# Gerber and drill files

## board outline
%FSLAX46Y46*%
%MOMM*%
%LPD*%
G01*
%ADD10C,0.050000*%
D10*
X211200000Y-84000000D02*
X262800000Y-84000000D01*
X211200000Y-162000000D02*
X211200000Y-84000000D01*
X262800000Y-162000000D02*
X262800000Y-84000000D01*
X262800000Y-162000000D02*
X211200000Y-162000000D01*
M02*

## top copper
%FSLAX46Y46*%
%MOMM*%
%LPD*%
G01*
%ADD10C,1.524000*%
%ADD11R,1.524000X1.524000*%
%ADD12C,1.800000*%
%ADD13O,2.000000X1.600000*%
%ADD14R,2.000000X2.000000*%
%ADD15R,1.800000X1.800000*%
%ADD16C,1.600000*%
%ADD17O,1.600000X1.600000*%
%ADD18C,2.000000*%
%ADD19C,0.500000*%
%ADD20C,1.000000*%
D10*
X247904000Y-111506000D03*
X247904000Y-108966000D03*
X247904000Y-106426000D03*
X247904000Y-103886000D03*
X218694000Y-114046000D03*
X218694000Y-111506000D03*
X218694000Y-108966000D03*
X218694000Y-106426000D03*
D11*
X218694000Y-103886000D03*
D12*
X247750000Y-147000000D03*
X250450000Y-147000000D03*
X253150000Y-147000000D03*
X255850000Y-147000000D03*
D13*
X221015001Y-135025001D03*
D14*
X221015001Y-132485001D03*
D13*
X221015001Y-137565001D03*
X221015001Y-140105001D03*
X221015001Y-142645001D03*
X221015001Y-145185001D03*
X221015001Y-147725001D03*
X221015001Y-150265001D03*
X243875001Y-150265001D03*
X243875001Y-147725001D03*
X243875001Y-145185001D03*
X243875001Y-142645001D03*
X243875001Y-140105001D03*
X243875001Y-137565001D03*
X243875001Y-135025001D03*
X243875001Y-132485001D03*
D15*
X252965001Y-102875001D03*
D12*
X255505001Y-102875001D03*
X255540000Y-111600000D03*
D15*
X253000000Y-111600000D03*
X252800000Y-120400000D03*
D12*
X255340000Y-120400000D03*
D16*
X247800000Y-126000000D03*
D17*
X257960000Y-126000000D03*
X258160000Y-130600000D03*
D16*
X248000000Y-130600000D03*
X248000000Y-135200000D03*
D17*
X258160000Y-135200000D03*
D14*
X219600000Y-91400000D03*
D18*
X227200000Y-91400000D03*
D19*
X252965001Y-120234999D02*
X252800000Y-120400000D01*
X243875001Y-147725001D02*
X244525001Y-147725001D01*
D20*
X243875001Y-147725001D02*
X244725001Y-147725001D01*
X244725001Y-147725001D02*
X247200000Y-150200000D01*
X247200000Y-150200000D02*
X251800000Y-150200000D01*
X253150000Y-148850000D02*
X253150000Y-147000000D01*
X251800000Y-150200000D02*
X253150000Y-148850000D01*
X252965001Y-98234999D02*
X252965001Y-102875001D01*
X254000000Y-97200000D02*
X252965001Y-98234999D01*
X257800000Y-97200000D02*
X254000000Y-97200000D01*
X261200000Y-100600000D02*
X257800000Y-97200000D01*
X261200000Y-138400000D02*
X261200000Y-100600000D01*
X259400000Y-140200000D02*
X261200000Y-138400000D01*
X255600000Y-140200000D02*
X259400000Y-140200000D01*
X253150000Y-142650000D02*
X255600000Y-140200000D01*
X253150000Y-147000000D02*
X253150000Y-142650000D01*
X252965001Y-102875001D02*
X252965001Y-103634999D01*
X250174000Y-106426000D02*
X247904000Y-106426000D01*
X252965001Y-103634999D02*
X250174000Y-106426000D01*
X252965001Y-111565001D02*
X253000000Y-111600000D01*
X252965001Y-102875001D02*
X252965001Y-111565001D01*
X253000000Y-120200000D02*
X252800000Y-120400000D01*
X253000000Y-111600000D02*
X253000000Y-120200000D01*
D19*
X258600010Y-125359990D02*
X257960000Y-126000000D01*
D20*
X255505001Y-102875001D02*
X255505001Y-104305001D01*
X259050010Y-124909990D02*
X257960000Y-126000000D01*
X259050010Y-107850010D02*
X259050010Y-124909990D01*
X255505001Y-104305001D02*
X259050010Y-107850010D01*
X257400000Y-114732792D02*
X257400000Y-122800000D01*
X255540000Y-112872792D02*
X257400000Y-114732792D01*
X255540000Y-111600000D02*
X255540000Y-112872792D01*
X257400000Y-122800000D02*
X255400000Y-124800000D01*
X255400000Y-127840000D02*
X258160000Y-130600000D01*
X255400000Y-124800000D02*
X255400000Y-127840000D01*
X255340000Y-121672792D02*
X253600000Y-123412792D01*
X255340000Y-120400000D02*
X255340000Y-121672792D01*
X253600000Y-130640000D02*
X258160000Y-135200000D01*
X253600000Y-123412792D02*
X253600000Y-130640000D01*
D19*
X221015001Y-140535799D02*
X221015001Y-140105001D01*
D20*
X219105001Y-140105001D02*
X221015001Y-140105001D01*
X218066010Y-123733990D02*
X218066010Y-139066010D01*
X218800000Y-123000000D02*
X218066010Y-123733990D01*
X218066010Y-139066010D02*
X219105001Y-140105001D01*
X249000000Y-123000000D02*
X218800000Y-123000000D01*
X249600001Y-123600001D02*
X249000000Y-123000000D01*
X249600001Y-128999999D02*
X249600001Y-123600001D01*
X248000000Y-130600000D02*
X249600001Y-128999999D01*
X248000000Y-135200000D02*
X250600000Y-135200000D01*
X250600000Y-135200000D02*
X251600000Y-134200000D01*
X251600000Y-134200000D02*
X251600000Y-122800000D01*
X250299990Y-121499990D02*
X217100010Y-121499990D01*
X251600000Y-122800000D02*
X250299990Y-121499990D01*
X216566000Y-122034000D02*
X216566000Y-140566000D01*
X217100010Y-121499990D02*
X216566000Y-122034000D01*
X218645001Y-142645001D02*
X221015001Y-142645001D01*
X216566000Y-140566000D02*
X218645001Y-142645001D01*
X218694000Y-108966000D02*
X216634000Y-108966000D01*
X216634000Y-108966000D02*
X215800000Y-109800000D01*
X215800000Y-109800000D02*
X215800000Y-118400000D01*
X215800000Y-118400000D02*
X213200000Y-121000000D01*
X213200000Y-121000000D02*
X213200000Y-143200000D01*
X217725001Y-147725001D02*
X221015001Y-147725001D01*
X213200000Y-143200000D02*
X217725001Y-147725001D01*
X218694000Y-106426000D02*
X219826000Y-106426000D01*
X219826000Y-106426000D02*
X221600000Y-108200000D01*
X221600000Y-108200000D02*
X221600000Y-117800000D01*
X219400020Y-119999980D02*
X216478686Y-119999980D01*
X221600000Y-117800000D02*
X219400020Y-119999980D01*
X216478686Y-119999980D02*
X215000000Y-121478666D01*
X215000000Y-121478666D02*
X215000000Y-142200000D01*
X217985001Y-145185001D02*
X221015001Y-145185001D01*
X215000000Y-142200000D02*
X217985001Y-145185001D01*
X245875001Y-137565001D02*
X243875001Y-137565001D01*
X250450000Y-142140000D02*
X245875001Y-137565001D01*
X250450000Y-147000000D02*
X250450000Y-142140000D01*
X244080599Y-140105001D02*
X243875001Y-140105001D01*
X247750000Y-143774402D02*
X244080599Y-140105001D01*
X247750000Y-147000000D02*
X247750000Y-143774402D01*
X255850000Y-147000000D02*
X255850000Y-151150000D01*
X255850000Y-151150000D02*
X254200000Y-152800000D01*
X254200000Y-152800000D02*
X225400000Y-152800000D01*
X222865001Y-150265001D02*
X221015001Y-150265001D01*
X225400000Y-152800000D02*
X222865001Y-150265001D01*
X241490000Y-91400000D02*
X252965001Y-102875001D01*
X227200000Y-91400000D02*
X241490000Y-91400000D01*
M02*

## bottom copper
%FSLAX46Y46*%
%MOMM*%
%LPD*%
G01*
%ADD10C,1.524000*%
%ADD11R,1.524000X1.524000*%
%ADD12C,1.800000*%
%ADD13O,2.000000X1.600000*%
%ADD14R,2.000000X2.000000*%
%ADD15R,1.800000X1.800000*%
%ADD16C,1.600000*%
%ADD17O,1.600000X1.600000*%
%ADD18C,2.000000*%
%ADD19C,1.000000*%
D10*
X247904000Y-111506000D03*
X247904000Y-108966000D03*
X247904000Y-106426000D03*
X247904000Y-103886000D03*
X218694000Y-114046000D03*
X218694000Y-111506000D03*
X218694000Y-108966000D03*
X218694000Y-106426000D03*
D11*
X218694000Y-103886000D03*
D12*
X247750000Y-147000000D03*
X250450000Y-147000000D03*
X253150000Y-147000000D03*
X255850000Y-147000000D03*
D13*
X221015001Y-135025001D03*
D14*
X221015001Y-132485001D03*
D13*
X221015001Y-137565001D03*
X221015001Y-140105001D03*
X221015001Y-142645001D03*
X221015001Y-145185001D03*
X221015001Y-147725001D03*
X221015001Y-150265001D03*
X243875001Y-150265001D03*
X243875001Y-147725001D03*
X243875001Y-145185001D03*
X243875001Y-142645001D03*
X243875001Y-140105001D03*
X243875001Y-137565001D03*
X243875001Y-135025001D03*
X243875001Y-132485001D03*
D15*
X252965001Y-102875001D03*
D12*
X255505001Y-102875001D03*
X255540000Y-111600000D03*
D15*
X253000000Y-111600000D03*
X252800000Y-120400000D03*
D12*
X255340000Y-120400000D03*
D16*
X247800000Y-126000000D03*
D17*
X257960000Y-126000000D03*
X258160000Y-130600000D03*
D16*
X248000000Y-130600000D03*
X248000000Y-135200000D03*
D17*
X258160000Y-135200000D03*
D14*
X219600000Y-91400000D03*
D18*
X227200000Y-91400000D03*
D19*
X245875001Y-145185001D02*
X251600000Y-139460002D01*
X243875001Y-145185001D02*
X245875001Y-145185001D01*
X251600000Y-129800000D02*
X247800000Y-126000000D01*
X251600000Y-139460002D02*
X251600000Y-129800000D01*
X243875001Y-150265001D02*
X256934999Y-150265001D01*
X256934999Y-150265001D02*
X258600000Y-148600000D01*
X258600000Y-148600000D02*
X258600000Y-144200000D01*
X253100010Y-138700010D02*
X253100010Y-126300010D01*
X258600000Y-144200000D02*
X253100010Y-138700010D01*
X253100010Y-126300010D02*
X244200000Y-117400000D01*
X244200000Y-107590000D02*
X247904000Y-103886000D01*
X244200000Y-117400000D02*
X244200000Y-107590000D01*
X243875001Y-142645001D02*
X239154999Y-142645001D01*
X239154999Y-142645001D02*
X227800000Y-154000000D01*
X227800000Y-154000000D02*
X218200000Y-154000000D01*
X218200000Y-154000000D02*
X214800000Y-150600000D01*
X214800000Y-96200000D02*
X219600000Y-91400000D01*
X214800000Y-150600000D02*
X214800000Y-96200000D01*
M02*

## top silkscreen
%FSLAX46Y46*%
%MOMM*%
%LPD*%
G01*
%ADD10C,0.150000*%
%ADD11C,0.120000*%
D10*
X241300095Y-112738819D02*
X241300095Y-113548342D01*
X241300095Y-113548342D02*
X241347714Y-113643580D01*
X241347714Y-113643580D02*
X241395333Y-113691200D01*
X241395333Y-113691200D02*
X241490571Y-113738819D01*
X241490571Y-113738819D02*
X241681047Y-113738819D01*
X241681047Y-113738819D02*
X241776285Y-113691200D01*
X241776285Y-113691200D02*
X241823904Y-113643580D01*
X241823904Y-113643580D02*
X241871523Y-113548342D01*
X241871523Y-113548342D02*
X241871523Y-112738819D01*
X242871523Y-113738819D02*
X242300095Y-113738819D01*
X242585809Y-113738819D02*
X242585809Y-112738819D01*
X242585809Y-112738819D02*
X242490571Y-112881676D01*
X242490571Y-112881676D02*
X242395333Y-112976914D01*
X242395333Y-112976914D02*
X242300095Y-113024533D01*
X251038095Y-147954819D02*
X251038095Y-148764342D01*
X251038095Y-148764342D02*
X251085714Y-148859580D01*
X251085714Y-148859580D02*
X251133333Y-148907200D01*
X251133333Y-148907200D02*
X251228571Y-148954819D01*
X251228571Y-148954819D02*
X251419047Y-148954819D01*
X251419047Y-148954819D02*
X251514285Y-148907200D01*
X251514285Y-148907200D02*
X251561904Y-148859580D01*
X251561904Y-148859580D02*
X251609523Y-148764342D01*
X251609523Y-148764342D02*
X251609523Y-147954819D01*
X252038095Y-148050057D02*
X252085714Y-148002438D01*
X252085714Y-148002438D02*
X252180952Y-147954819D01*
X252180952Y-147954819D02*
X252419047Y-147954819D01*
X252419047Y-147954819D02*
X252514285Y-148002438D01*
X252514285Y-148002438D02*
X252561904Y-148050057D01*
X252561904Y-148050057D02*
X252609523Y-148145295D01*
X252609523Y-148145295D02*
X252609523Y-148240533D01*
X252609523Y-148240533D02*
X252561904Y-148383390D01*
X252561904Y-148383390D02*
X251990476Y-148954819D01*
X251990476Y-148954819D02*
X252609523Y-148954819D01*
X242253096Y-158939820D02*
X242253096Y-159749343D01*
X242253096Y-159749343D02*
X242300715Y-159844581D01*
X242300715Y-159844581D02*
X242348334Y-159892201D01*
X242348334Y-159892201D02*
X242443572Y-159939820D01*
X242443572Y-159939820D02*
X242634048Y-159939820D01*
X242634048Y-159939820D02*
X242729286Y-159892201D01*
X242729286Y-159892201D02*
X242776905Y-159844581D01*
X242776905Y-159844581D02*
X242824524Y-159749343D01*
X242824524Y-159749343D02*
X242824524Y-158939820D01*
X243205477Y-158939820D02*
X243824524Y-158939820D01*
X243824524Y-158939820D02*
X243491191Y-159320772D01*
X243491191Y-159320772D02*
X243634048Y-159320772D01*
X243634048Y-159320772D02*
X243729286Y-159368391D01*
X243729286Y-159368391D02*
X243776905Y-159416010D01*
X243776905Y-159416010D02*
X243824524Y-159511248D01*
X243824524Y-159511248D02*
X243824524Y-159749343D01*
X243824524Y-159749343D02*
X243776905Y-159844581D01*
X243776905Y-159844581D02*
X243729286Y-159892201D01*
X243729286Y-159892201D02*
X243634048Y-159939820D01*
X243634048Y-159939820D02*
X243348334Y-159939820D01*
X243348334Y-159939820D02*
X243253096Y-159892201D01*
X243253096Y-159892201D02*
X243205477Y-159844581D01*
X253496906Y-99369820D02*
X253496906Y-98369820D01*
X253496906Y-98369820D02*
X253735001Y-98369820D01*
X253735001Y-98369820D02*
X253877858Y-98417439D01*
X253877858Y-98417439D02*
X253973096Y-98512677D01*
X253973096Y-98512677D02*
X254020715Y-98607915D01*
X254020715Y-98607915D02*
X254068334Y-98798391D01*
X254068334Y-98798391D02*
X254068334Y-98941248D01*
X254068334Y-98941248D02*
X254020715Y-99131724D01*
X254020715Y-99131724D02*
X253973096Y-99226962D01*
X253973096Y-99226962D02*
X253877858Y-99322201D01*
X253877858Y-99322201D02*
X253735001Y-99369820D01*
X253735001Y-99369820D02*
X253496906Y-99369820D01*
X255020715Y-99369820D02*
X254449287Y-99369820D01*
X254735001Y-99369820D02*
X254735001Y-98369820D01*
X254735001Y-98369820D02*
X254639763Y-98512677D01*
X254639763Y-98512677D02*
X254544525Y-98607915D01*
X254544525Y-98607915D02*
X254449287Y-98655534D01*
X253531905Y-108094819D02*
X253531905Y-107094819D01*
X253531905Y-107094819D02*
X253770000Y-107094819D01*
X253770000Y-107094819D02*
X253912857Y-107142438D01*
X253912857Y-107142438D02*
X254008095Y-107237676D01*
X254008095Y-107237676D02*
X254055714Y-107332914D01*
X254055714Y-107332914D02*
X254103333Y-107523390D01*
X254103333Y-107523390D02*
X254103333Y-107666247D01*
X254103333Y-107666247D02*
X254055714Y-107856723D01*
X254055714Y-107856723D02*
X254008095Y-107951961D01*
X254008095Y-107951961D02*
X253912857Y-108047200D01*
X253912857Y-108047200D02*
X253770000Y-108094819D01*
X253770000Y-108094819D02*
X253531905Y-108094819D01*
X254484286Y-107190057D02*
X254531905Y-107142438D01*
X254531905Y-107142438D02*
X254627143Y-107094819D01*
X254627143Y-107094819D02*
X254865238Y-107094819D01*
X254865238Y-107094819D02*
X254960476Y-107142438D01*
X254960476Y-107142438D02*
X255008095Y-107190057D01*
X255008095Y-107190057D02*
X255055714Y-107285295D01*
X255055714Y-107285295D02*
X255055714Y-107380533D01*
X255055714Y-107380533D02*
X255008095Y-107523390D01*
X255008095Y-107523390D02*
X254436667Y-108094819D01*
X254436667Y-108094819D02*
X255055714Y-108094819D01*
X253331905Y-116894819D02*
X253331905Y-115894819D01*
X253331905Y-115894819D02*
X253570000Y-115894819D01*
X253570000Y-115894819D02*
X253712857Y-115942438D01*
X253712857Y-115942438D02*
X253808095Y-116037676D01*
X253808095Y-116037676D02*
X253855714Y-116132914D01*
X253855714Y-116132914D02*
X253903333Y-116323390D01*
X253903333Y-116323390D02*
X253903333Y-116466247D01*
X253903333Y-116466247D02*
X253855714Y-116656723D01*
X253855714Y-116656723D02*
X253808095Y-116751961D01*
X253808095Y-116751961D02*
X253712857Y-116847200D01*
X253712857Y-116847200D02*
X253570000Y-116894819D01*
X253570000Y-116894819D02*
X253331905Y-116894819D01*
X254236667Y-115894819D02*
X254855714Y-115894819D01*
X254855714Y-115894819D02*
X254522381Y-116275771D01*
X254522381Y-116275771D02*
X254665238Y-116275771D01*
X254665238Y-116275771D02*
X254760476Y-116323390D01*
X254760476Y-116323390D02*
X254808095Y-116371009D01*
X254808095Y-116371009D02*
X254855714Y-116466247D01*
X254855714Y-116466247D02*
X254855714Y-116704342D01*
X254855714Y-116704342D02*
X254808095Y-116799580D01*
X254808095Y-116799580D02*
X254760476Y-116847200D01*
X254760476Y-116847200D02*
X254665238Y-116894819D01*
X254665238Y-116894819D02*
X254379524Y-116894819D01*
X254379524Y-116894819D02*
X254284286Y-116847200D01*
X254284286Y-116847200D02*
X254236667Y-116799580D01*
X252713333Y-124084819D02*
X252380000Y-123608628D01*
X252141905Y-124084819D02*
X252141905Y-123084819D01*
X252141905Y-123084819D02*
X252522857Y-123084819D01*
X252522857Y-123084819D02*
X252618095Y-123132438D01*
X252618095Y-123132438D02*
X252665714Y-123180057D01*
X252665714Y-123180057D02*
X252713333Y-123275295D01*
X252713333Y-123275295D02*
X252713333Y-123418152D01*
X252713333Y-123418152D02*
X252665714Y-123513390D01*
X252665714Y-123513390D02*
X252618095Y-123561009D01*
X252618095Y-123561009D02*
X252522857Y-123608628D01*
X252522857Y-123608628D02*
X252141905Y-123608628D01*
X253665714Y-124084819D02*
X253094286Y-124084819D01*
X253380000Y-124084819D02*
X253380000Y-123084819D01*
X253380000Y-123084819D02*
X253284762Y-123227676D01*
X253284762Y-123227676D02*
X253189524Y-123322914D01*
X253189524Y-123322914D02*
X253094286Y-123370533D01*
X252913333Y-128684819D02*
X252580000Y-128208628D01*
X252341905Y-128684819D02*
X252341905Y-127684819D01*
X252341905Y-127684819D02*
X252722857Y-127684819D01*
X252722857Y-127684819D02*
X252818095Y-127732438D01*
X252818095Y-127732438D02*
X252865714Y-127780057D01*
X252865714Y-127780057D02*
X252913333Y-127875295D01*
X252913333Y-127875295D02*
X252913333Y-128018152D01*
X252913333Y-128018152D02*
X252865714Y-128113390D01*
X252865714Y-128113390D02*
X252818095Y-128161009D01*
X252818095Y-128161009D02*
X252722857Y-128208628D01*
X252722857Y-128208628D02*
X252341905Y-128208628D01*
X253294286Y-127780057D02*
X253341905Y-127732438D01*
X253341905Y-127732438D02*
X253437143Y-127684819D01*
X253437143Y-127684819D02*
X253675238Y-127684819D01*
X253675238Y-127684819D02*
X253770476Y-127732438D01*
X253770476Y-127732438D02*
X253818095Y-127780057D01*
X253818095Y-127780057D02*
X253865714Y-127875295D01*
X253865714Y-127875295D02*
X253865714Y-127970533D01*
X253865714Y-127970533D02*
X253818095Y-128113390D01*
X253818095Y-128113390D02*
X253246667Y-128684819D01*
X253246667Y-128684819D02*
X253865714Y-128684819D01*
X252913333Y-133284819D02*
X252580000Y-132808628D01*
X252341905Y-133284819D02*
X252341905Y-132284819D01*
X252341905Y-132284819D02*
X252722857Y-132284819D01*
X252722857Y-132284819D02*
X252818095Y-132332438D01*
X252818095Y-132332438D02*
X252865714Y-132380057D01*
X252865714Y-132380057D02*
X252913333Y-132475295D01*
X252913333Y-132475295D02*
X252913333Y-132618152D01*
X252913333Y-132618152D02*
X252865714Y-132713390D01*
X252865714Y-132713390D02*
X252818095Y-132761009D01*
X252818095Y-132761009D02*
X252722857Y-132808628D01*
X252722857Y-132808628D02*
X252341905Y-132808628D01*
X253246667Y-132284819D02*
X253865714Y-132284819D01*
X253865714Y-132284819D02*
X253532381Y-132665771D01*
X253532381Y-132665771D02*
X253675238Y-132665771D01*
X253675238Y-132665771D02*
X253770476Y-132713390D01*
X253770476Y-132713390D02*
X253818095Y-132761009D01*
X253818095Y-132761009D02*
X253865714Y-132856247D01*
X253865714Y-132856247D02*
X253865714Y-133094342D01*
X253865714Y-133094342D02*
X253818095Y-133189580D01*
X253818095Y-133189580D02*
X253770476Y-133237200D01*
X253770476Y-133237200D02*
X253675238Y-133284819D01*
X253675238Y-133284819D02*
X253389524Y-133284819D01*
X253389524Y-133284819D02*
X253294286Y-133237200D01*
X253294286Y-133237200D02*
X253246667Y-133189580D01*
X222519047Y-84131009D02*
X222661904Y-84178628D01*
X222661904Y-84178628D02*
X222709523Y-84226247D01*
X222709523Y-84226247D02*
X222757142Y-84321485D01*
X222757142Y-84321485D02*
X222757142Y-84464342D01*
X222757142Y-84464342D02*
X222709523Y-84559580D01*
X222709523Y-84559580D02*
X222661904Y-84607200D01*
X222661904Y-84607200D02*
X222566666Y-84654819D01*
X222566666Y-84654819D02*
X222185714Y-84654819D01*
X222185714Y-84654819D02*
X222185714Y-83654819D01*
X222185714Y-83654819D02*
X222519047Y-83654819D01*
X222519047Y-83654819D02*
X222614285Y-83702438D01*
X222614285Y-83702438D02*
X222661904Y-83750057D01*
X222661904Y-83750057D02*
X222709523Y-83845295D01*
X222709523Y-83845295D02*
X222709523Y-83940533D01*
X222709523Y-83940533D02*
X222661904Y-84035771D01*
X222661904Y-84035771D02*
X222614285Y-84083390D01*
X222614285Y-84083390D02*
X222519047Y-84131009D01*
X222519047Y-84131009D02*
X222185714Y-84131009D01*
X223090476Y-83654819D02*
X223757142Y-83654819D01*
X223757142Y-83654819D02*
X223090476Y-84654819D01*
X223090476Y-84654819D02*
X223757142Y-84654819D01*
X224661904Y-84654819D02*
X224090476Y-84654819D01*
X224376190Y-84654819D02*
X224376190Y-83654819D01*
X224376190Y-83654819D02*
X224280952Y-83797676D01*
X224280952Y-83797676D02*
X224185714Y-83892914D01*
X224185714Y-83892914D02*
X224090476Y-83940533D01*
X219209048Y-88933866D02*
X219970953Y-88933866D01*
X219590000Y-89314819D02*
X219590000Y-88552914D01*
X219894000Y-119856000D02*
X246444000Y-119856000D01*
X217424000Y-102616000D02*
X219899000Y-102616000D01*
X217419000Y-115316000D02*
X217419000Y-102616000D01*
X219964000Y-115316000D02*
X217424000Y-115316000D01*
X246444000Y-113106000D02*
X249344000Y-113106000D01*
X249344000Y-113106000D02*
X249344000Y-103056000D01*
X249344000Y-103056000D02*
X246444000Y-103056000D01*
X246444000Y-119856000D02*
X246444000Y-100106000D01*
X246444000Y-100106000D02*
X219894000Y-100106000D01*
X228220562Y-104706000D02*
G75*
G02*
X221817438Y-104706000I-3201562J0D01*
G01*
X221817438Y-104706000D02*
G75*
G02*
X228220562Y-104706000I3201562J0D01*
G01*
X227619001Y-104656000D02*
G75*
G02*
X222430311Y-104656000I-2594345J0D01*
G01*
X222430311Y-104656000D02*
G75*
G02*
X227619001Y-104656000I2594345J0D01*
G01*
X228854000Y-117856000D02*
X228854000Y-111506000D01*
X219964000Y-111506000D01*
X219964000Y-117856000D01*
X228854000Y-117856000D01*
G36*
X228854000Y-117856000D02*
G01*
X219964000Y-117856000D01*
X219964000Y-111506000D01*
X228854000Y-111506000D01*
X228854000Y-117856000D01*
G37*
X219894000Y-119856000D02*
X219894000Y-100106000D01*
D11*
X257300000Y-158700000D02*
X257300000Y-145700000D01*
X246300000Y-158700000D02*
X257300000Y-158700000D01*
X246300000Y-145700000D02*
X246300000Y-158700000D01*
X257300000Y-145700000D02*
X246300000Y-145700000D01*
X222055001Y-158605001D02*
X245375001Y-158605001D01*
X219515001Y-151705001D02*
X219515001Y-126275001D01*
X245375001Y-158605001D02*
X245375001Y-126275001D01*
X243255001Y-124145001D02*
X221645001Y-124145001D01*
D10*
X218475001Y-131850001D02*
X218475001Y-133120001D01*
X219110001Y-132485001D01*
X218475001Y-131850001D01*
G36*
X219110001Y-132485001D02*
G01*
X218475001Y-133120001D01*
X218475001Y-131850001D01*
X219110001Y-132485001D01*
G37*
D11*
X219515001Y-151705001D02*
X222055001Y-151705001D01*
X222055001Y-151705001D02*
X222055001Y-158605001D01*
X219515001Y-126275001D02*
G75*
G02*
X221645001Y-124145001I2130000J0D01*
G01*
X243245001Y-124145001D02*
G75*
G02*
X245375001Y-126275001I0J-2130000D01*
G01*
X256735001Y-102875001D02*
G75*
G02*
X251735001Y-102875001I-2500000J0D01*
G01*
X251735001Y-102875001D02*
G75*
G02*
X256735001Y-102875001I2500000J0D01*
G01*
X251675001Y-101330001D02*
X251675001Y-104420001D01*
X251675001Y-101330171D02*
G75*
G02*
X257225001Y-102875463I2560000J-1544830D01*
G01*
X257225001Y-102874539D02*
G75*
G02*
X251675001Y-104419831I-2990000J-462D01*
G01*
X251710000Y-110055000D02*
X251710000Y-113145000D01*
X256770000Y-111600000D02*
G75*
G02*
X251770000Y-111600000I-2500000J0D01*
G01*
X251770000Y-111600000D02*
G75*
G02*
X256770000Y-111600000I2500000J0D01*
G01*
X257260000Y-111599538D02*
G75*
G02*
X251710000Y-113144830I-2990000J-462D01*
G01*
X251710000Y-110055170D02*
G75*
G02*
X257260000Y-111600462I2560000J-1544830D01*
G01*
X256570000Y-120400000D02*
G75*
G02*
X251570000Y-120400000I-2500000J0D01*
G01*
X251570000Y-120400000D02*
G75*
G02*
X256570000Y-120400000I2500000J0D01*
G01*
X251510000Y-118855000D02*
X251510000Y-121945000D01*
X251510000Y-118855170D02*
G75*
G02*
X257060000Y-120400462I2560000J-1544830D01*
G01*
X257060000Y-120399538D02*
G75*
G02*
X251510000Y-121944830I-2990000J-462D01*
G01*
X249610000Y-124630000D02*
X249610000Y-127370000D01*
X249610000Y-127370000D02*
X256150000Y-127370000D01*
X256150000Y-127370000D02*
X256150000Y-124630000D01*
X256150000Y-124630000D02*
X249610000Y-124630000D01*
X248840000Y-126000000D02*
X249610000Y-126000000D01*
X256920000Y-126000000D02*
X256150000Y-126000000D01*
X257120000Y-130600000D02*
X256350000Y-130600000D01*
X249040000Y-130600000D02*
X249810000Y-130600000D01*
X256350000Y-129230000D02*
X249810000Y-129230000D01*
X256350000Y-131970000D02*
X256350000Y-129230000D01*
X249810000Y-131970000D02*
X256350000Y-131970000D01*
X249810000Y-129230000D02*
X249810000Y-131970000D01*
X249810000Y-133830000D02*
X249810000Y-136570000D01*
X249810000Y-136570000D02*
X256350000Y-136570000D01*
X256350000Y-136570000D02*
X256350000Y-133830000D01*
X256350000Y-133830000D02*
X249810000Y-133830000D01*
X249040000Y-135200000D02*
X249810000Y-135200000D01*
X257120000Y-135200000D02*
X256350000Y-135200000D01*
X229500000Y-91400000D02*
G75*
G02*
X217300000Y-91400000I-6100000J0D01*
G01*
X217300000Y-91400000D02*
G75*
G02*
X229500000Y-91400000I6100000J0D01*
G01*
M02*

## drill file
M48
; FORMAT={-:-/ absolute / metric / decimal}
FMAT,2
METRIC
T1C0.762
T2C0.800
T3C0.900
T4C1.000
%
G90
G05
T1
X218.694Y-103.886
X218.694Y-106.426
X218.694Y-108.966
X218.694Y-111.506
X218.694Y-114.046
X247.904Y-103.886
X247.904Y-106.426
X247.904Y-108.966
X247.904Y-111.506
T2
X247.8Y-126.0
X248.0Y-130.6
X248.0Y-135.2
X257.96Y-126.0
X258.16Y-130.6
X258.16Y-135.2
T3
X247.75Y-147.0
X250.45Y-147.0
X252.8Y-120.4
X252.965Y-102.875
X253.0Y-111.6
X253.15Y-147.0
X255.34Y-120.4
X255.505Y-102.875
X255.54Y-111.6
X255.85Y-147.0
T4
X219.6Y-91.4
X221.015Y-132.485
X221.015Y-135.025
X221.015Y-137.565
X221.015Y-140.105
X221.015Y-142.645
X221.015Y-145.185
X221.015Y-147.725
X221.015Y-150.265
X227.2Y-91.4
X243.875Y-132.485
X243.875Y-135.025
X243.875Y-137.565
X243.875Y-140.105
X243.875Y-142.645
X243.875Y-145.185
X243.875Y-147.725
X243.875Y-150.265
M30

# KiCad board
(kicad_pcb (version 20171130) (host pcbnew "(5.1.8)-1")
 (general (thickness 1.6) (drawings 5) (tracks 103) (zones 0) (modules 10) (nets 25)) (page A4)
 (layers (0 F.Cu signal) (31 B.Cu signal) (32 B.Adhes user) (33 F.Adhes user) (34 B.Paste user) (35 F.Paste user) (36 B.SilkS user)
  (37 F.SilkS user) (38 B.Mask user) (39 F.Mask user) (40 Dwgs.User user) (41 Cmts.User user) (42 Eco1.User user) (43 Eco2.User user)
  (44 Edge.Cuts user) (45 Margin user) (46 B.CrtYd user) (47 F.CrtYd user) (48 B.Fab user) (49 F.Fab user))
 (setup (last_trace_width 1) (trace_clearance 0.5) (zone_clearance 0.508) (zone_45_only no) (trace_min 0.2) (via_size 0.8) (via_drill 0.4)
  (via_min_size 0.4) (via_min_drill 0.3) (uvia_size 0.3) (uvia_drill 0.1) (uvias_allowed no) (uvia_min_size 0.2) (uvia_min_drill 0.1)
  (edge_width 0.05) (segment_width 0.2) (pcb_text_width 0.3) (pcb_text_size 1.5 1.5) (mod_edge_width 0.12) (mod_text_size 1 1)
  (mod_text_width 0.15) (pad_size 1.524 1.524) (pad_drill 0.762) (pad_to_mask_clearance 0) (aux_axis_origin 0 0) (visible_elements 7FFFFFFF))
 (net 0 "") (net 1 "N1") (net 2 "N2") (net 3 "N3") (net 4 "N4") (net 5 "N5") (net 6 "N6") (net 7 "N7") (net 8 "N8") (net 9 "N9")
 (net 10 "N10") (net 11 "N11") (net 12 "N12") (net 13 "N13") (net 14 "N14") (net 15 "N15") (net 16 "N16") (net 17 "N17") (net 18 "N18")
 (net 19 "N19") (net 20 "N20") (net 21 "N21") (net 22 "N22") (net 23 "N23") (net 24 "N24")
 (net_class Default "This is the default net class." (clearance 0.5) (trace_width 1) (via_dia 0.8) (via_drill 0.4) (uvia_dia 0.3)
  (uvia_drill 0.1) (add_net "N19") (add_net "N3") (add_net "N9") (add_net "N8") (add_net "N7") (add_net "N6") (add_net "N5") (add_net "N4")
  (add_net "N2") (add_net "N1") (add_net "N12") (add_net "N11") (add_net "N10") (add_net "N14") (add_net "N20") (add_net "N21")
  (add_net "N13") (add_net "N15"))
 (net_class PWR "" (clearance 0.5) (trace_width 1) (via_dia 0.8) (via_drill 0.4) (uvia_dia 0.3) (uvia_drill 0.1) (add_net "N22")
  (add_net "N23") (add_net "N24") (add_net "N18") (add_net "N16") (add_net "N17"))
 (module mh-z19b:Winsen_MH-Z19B (layer F.Cu) (at 218.694 117.856 180)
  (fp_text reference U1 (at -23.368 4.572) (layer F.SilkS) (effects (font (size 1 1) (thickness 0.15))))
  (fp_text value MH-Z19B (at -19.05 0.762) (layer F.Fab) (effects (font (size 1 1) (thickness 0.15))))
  (fp_line (start -1.2 -2) (end -27.75 -2) (layer F.SilkS) (width 0.15))
  (fp_line (start 1.27 15.24) (end -1.205 15.24) (layer F.SilkS) (width 0.15))
  (fp_line (start 1.275 2.54) (end 1.275 15.24) (layer F.SilkS) (width 0.15))
  (fp_line (start -1.27 2.54) (end 1.27 2.54) (layer F.SilkS) (width 0.15))
  (fp_line (start -27.75 4.75) (end -30.65 4.75) (layer F.SilkS) (width 0.15))
  (fp_line (start -30.65 4.75) (end -30.65 14.8) (layer F.SilkS) (width 0.15))
  (fp_line (start -30.65 14.8) (end -27.75 14.8) (layer F.SilkS) (width 0.15))
  (fp_line (start -27.75 -2) (end -27.75 17.75) (layer F.SilkS) (width 0.15))
  (fp_line (start -27.75 17.75) (end -1.2 17.75) (layer F.SilkS) (width 0.15))
  (fp_circle (center -6.325 13.15) (end -9.425 12.35) (layer F.SilkS) (width 0.15))
  (fp_circle (center -6.330656 13.2) (end -8.530656 11.825) (layer F.SilkS) (width 0.15))
  (fp_poly (pts (xy -10.16 0) (xy -10.16 6.35) (xy -1.27 6.35) (xy -1.27 0)) (layer F.SilkS) (width 0.15))
  (fp_line (start -1.2 -2) (end -1.2 17.75) (layer F.SilkS) (width 0.15))
  (pad 9 thru_hole circle (at -29.21 6.35 180) (size 1.524 1.524) (drill 0.762) (layers *.Cu *.Mask) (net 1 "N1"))
  (pad 8 thru_hole circle (at -29.21 8.89 180) (size 1.524 1.524) (drill 0.762) (layers *.Cu *.Mask) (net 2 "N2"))
  (pad 7 thru_hole circle (at -29.21 11.43 180) (size 1.524 1.524) (drill 0.762) (layers *.Cu *.Mask) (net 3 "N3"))
  (pad 6 thru_hole circle (at -29.21 13.97 180) (size 1.524 1.524) (drill 0.762) (layers *.Cu *.Mask) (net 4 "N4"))
  (pad 5 thru_hole circle (at 0 3.81 180) (size 1.524 1.524) (drill 0.762) (layers *.Cu *.Mask) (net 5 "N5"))
  (pad 4 thru_hole circle (at 0 6.35 180) (size 1.524 1.524) (drill 0.762) (layers *.Cu *.Mask) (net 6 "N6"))
  (pad 3 thru_hole circle (at 0 8.89 180) (size 1.524 1.524) (drill 0.762) (layers *.Cu *.Mask) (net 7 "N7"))
  (pad 2 thru_hole circle (at 0 11.43 180) (size 1.524 1.524) (drill 0.762) (layers *.Cu *.Mask) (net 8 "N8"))
  (pad 1 thru_hole rect (at 0 13.97 180) (size 1.524 1.524) (drill 0.762) (layers *.Cu *.Mask) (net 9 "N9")))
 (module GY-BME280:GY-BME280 (layer F.Cu) (at 251.8 149 180)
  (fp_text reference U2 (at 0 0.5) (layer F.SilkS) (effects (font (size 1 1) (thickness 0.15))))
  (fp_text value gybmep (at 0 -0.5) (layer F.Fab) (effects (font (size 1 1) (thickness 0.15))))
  (fp_line (start -5.5 -9.7) (end -5.5 3.3) (layer F.SilkS) (width 0.12))
  (fp_line (start 5.5 -9.7) (end -5.5 -9.7) (layer F.SilkS) (width 0.12))
  (fp_line (start 5.5 3.3) (end 5.5 -9.7) (layer F.SilkS) (width 0.12))
  (fp_line (start -5.5 3.3) (end 5.5 3.3) (layer F.SilkS) (width 0.12))
  (pad 4 thru_hole circle (at 4.05 2 180) (size 1.8 1.8) (drill 0.9) (layers *.Cu *.Mask) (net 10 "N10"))
  (pad 3 thru_hole circle (at 1.35 2 180) (size 1.8 1.8) (drill 0.9) (layers *.Cu *.Mask) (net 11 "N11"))
  (pad 2 thru_hole circle (at -1.35 2 180) (size 1.8 1.8) (drill 0.9) (layers *.Cu *.Mask) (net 3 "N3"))
  (pad 1 thru_hole circle (at -4.05 2 180) (size 1.8 1.8) (drill 0.9) (layers *.Cu *.Mask) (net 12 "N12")))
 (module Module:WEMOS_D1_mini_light (layer F.Cu) (at 221.015001 132.485001)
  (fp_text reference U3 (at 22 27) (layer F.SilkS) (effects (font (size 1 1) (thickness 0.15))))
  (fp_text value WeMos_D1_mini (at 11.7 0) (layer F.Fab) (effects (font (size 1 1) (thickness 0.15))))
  (fp_line (start 1.04 26.12) (end 24.36 26.12) (layer F.SilkS) (width 0.12))
  (fp_line (start -1.5 19.22) (end -1.5 -6.21) (layer F.SilkS) (width 0.12))
  (fp_line (start 24.36 26.12) (end 24.36 -6.21) (layer F.SilkS) (width 0.12))
  (fp_line (start 22.24 -8.34) (end 0.63 -8.34) (layer F.SilkS) (width 0.12))
  (fp_poly (pts (xy -2.54 -0.635) (xy -2.54 0.635) (xy -1.905 0)) (layer F.SilkS) (width 0.15))
  (fp_line (start -1.5 19.22) (end 1.04 19.22) (layer F.SilkS) (width 0.12))
  (fp_line (start 1.04 19.22) (end 1.04 26.12) (layer F.SilkS) (width 0.12))
  (fp_arc (start 0.63 -6.21) (end 0.63 -8.34) (angle -90) (layer F.SilkS) (width 0.12))
  (fp_arc (start 22.23 -6.21) (end 24.36 -6.21) (angle -90) (layer F.SilkS) (width 0.12))
  (pad 2 thru_hole oval (at 0 2.54) (size 2 1.6) (drill 1) (layers *.Cu *.Mask) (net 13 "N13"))
  (pad 1 thru_hole rect (at 0 0) (size 2 2) (drill 1) (layers *.Cu *.Mask) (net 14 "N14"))
  (pad 3 thru_hole oval (at 0 5.08) (size 2 1.6) (drill 1) (layers *.Cu *.Mask) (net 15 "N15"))
  (pad 4 thru_hole oval (at 0 7.62) (size 2 1.6) (drill 1) (layers *.Cu *.Mask) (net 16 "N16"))
  (pad 5 thru_hole oval (at 0 10.16) (size 2 1.6) (drill 1) (layers *.Cu *.Mask) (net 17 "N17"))
  (pad 6 thru_hole oval (at 0 12.7) (size 2 1.6) (drill 1) (layers *.Cu *.Mask) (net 8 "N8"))
  (pad 7 thru_hole oval (at 0 15.24) (size 2 1.6) (drill 1) (layers *.Cu *.Mask) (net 7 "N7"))
  (pad 8 thru_hole oval (at 0 17.78) (size 2 1.6) (drill 1) (layers *.Cu *.Mask) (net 12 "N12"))
  (pad 9 thru_hole oval (at 22.86 17.78) (size 2 1.6) (drill 1) (layers *.Cu *.Mask) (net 4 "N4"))
  (pad 10 thru_hole oval (at 22.86 15.24) (size 2 1.6) (drill 1) (layers *.Cu *.Mask) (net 3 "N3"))
  (pad 11 thru_hole oval (at 22.86 12.7) (size 2 1.6) (drill 1) (layers *.Cu *.Mask) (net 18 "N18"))
  (pad 12 thru_hole oval (at 22.86 10.16) (size 2 1.6) (drill 1) (layers *.Cu *.Mask) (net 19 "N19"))
  (pad 13 thru_hole oval (at 22.86 7.62) (size 2 1.6) (drill 1) (layers *.Cu *.Mask) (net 10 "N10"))
  (pad 14 thru_hole oval (at 22.86 5.08) (size 2 1.6) (drill 1) (layers *.Cu *.Mask) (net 11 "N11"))
  (pad 15 thru_hole oval (at 22.86 2.54) (size 2 1.6) (drill 1) (layers *.Cu *.Mask) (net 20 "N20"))
  (pad 16 thru_hole oval (at 22.86 0) (size 2 1.6) (drill 1) (layers *.Cu *.Mask) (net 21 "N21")))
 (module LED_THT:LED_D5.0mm (layer F.Cu) (at 252.965001 102.875001)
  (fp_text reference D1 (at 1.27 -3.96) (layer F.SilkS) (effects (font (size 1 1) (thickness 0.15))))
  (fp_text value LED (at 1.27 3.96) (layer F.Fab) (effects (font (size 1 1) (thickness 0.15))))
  (fp_circle (center 1.27 0) (end 3.77 0) (layer F.SilkS) (width 0.12))
  (fp_line (start -1.29 -1.545) (end -1.29 1.545) (layer F.SilkS) (width 0.12))
  (fp_arc (start 1.27 0) (end -1.29 -1.54483) (angle 148.9) (layer F.SilkS) (width 0.12))
  (fp_arc (start 1.27 0) (end -1.29 1.54483) (angle -148.9) (layer F.SilkS) (width 0.12))
  (pad 1 thru_hole rect (at 0 0) (size 1.8 1.8) (drill 0.9) (layers *.Cu *.Mask) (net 3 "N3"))
  (pad 2 thru_hole circle (at 2.54 0) (size 1.8 1.8) (drill 0.9) (layers *.Cu *.Mask) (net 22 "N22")))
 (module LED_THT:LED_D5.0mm (layer F.Cu) (at 253 111.6)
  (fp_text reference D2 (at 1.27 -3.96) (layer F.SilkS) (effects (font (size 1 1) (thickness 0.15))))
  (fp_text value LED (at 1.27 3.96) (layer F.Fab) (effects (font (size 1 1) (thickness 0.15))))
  (fp_line (start -1.29 -1.545) (end -1.29 1.545) (layer F.SilkS) (width 0.12))
  (fp_circle (center 1.27 0) (end 3.77 0) (layer F.SilkS) (width 0.12))
  (fp_arc (start 1.27 0) (end -1.29 1.54483) (angle -148.9) (layer F.SilkS) (width 0.12))
  (fp_arc (start 1.27 0) (end -1.29 -1.54483) (angle 148.9) (layer F.SilkS) (width 0.12))
  (pad 2 thru_hole circle (at 2.54 0) (size 1.8 1.8) (drill 0.9) (layers *.Cu *.Mask) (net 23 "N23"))
  (pad 1 thru_hole rect (at 0 0) (size 1.8 1.8) (drill 0.9) (layers *.Cu *.Mask) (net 3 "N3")))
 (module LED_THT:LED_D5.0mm (layer F.Cu) (at 252.8 120.4)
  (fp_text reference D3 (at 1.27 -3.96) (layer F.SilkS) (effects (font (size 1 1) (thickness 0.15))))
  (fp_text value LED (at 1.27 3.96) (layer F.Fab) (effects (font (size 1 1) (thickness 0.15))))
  (fp_circle (center 1.27 0) (end 3.77 0) (layer F.SilkS) (width 0.12))
  (fp_line (start -1.29 -1.545) (end -1.29 1.545) (layer F.SilkS) (width 0.12))
  (fp_arc (start 1.27 0) (end -1.29 -1.54483) (angle 148.9) (layer F.SilkS) (width 0.12))
  (fp_arc (start 1.27 0) (end -1.29 1.54483) (angle -148.9) (layer F.SilkS) (width 0.12))
  (pad 1 thru_hole rect (at 0 0) (size 1.8 1.8) (drill 0.9) (layers *.Cu *.Mask) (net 3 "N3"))
  (pad 2 thru_hole circle (at 2.54 0) (size 1.8 1.8) (drill 0.9) (layers *.Cu *.Mask) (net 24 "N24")))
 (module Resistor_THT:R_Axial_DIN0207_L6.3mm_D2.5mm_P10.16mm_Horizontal (layer F.Cu) (at 247.8 126)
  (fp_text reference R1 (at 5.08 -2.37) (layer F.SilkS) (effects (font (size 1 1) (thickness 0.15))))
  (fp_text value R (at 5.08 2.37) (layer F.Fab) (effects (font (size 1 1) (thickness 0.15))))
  (fp_line (start 1.81 -1.37) (end 1.81 1.37) (layer F.SilkS) (width 0.12))
  (fp_line (start 1.81 1.37) (end 8.35 1.37) (layer F.SilkS) (width 0.12))
  (fp_line (start 8.35 1.37) (end 8.35 -1.37) (layer F.SilkS) (width 0.12))
  (fp_line (start 8.35 -1.37) (end 1.81 -1.37) (layer F.SilkS) (width 0.12))
  (fp_line (start 1.04 0) (end 1.81 0) (layer F.SilkS) (width 0.12))
  (fp_line (start 9.12 0) (end 8.35 0) (layer F.SilkS) (width 0.12))
  (pad 1 thru_hole circle (at 0 0) (size 1.6 1.6) (drill 0.8) (layers *.Cu *.Mask) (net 18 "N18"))
  (pad 2 thru_hole oval (at 10.16 0) (size 1.6 1.6) (drill 0.8) (layers *.Cu *.Mask) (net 22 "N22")))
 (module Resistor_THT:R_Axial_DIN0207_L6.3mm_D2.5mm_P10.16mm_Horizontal (layer F.Cu) (at 248 130.6)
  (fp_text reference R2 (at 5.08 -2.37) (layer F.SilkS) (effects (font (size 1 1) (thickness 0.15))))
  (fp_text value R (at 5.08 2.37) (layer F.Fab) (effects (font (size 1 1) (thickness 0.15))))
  (fp_line (start 9.12 0) (end 8.35 0) (layer F.SilkS) (width 0.12))
  (fp_line (start 1.04 0) (end 1.81 0) (layer F.SilkS) (width 0.12))
  (fp_line (start 8.35 -1.37) (end 1.81 -1.37) (layer F.SilkS) (width 0.12))
  (fp_line (start 8.35 1.37) (end 8.35 -1.37) (layer F.SilkS) (width 0.12))
  (fp_line (start 1.81 1.37) (end 8.35 1.37) (layer F.SilkS) (width 0.12))
  (fp_line (start 1.81 -1.37) (end 1.81 1.37) (layer F.SilkS) (width 0.12))
  (pad 2 thru_hole oval (at 10.16 0) (size 1.6 1.6) (drill 0.8) (layers *.Cu *.Mask) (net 23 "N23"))
  (pad 1 thru_hole circle (at 0 0) (size 1.6 1.6) (drill 0.8) (layers *.Cu *.Mask) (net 16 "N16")))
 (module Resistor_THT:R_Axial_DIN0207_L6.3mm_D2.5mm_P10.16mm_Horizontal (layer F.Cu) (at 248 135.2)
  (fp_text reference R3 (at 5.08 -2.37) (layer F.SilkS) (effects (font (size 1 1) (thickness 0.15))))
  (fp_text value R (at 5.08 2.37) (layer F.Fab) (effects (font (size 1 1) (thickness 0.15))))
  (fp_line (start 1.81 -1.37) (end 1.81 1.37) (layer F.SilkS) (width 0.12))
  (fp_line (start 1.81 1.37) (end 8.35 1.37) (layer F.SilkS) (width 0.12))
  (fp_line (start 8.35 1.37) (end 8.35 -1.37) (layer F.SilkS) (width 0.12))
  (fp_line (start 8.35 -1.37) (end 1.81 -1.37) (layer F.SilkS) (width 0.12))
  (fp_line (start 1.04 0) (end 1.81 0) (layer F.SilkS) (width 0.12))
  (fp_line (start 9.12 0) (end 8.35 0) (layer F.SilkS) (width 0.12))
  (pad 1 thru_hole circle (at 0 0) (size 1.6 1.6) (drill 0.8) (layers *.Cu *.Mask) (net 17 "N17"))
  (pad 2 thru_hole oval (at 10.16 0) (size 1.6 1.6) (drill 0.8) (layers *.Cu *.Mask) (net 24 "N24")))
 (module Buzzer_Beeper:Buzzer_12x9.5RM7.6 (layer F.Cu) (at 219.6 91.4)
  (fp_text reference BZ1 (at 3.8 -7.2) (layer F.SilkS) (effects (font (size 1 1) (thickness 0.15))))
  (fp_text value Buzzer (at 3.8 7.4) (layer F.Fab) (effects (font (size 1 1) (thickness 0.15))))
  (fp_circle (center 3.8 0) (end 9.9 0) (layer F.SilkS) (width 0.12))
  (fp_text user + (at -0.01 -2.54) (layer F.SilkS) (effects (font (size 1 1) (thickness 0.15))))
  (pad 1 thru_hole rect (at 0 0) (size 2 2) (drill 1) (layers *.Cu *.Mask) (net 19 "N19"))
  (pad 2 thru_hole circle (at 7.6 0) (size 2 2) (drill 1) (layers *.Cu *.Mask) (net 3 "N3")))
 (gr_line (start 211.2 84) (end 262.8 84) (layer Edge.Cuts) (width 0.05))
 (gr_line (start 211.2 162) (end 211.2 84) (layer Edge.Cuts) (width 0.05))
 (gr_line (start 262.8 162) (end 262.8 84) (layer Edge.Cuts) (width 0.05))
 (gr_line (start 262.8 162) (end 211.2 162) (layer Edge.Cuts) (width 0.05))
 (segment (start 252.965001 120.234999) (end 252.8 120.4) (width 0.5) (layer F.Cu) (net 3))
 (segment (start 243.875001 147.725001) (end 244.525001 147.725001) (width 0.5) (layer F.Cu) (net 3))
 (segment (start 243.875001 147.725001) (end 244.725001 147.725001) (width 1) (layer F.Cu) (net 3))
 (segment (start 244.725001 147.725001) (end 247.2 150.2) (width 1) (layer F.Cu) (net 3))
 (segment (start 247.2 150.2) (end 251.8 150.2) (width 1) (layer F.Cu) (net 3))
 (segment (start 253.15 148.85) (end 253.15 147) (width 1) (layer F.Cu) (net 3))
 (segment (start 251.8 150.2) (end 253.15 148.85) (width 1) (layer F.Cu) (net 3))
 (segment (start 252.965001 98.234999) (end 252.965001 102.875001) (width 1) (layer F.Cu) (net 3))
 (segment (start 254 97.2) (end 252.965001 98.234999) (width 1) (layer F.Cu) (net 3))
 (segment (start 257.8 97.2) (end 254 97.2) (width 1) (layer F.Cu) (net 3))
 (segment (start 261.2 100.6) (end 257.8 97.2) (width 1) (layer F.Cu) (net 3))
 (segment (start 261.2 138.4) (end 261.2 100.6) (width 1) (layer F.Cu) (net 3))
 (segment (start 259.4 140.2) (end 261.2 138.4) (width 1) (layer F.Cu) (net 3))
 (segment (start 255.6 140.2) (end 259.4 140.2) (width 1) (layer F.Cu) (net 3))
 (segment (start 253.15 142.65) (end 255.6 140.2) (width 1) (layer F.Cu) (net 3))
 (segment (start 253.15 147) (end 253.15 142.65) (width 1) (layer F.Cu) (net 3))
 (segment (start 252.965001 102.875001) (end 252.965001 103.634999) (width 1) (layer F.Cu) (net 3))
 (segment (start 250.174 106.426) (end 247.904 106.426) (width 1) (layer F.Cu) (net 3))
 (segment (start 252.965001 103.634999) (end 250.174 106.426) (width 1) (layer F.Cu) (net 3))
 (segment (start 252.965001 111.565001) (end 253 111.6) (width 1) (layer F.Cu) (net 3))
 (segment (start 252.965001 102.875001) (end 252.965001 111.565001) (width 1) (layer F.Cu) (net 3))
 (segment (start 253 120.2) (end 252.8 120.4) (width 1) (layer F.Cu) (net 3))
 (segment (start 253 111.6) (end 253 120.2) (width 1) (layer F.Cu) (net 3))
 (segment (start 258.60001 125.35999) (end 257.96 126) (width 0.5) (layer F.Cu) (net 22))
 (segment (start 255.505001 102.875001) (end 255.505001 104.305001) (width 1) (layer F.Cu) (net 22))
 (segment (start 259.05001 124.90999) (end 257.96 126) (width 1) (layer F.Cu) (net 22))
 (segment (start 259.05001 107.85001) (end 259.05001 124.90999) (width 1) (layer F.Cu) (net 22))
 (segment (start 255.505001 104.305001) (end 259.05001 107.85001) (width 1) (layer F.Cu) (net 22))
 (segment (start 257.4 114.732792) (end 257.4 122.8) (width 1) (layer F.Cu) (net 23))
 (segment (start 255.54 112.872792) (end 257.4 114.732792) (width 1) (layer F.Cu) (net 23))
 (segment (start 255.54 111.6) (end 255.54 112.872792) (width 1) (layer F.Cu) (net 23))
 (segment (start 257.4 122.8) (end 255.4 124.8) (width 1) (layer F.Cu) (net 23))
 (segment (start 255.4 127.84) (end 258.16 130.6) (width 1) (layer F.Cu) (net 23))
 (segment (start 255.4 124.8) (end 255.4 127.84) (width 1) (layer F.Cu) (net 23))
 (segment (start 255.34 121.672792) (end 253.6 123.412792) (width 1) (layer F.Cu) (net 24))
 (segment (start 255.34 120.4) (end 255.34 121.672792) (width 1) (layer F.Cu) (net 24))
 (segment (start 253.6 130.64) (end 258.16 135.2) (width 1) (layer F.Cu) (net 24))
 (segment (start 253.6 123.412792) (end 253.6 130.64) (width 1) (layer F.Cu) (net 24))
 (segment (start 245.875001 145.185001) (end 251.6 139.460002) (width 1) (layer B.Cu) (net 18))
 (segment (start 243.875001 145.185001) (end 245.875001 145.185001) (width 1) (layer B.Cu) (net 18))
 (segment (start 251.6 129.8) (end 247.8 126) (width 1) (layer B.Cu) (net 18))
 (segment (start 251.6 139.460002) (end 251.6 129.8) (width 1) (layer B.Cu) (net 18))
 (segment (start 221.015001 140.535799) (end 221.015001 140.105001) (width 0.5) (layer F.Cu) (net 16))
 (segment (start 219.105001 140.105001) (end 221.015001 140.105001) (width 1) (layer F.Cu) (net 16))
 (segment (start 218.06601 123.73399) (end 218.06601 139.06601) (width 1) (layer F.Cu) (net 16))
 (segment (start 218.8 123) (end 218.06601 123.73399) (width 1) (layer F.Cu) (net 16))
 (segment (start 218.06601 139.06601) (end 219.105001 140.105001) (width 1) (layer F.Cu) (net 16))
 (segment (start 249 123) (end 218.8 123) (width 1) (layer F.Cu) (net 16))
 (segment (start 249.600001 123.600001) (end 249 123) (width 1) (layer F.Cu) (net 16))
 (segment (start 249.600001 128.999999) (end 249.600001 123.600001) (width 1) (layer F.Cu) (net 16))
 (segment (start 248 130.6) (end 249.600001 128.999999) (width 1) (layer F.Cu) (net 16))
 (segment (start 248 135.2) (end 250.6 135.2) (width 1) (layer F.Cu) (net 17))
 (segment (start 250.6 135.2) (end 251.6 134.2) (width 1) (layer F.Cu) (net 17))
 (segment (start 251.6 134.2) (end 251.6 122.8) (width 1) (layer F.Cu) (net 17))
 (segment (start 250.29999 121.49999) (end 217.10001 121.49999) (width 1) (layer F.Cu) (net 17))
 (segment (start 251.6 122.8) (end 250.29999 121.49999) (width 1) (layer F.Cu) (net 17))
 (segment (start 216.566 122.034) (end 216.566 140.566) (width 1) (layer F.Cu) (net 17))
 (segment (start 217.10001 121.49999) (end 216.566 122.034) (width 1) (layer F.Cu) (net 17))
 (segment (start 218.645001 142.645001) (end 221.015001 142.645001) (width 1) (layer F.Cu) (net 17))
 (segment (start 216.566 140.566) (end 218.645001 142.645001) (width 1) (layer F.Cu) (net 17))
 (segment (start 243.875001 150.265001) (end 256.934999 150.265001) (width 1) (layer B.Cu) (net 4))
 (segment (start 256.934999 150.265001) (end 258.6 148.6) (width 1) (layer B.Cu) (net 4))
 (segment (start 258.6 148.6) (end 258.6 144.2) (width 1) (layer B.Cu) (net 4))
 (segment (start 253.10001 138.70001) (end 253.10001 126.30001) (width 1) (layer B.Cu) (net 4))
 (segment (start 258.6 144.2) (end 253.10001 138.70001) (width 1) (layer B.Cu) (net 4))
 (segment (start 253.10001 126.30001) (end 244.2 117.4) (width 1) (layer B.Cu) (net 4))
 (segment (start 244.2 107.59) (end 247.904 103.886) (width 1) (layer B.Cu) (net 4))
 (segment (start 244.2 117.4) (end 244.2 107.59) (width 1) (layer B.Cu) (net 4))
 (segment (start 218.694 108.966) (end 216.634 108.966) (width 1) (layer F.Cu) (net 7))
 (segment (start 216.634 108.966) (end 215.8 109.8) (width 1) (layer F.Cu) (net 7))
 (segment (start 215.8 109.8) (end 215.8 118.4) (width 1) (layer F.Cu) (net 7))
 (segment (start 215.8 118.4) (end 213.2 121) (width 1) (layer F.Cu) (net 7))
 (segment (start 213.2 121) (end 213.2 143.2) (width 1) (layer F.Cu) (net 7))
 (segment (start 217.725001 147.725001) (end 221.015001 147.725001) (width 1) (layer F.Cu) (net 7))
 (segment (start 213.2 143.2) (end 217.725001 147.725001) (width 1) (layer F.Cu) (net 7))
 (segment (start 218.694 106.426) (end 219.826 106.426) (width 1) (layer F.Cu) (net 8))
 (segment (start 219.826 106.426) (end 221.6 108.2) (width 1) (layer F.Cu) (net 8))
 (segment (start 221.6 108.2) (end 221.6 117.8) (width 1) (layer F.Cu) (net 8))
 (segment (start 219.40002 119.99998) (end 216.478686 119.99998) (width 1) (layer F.Cu) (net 8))
 (segment (start 221.6 117.8) (end 219.40002 119.99998) (width 1) (layer F.Cu) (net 8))
 (segment (start 216.478686 119.99998) (end 215 121.478666) (width 1) (layer F.Cu) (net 8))
 (segment (start 215 121.478666) (end 215 142.2) (width 1) (layer F.Cu) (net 8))
 (segment (start 217.985001 145.185001) (end 221.015001 145.185001) (width 1) (layer F.Cu) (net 8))
 (segment (start 215 142.2) (end 217.985001 145.185001) (width 1) (layer F.Cu) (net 8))
 (segment (start 245.875001 137.565001) (end 243.875001 137.565001) (width 1) (layer F.Cu) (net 11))
 (segment (start 250.45 142.14) (end 245.875001 137.565001) (width 1) (layer F.Cu) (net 11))
 (segment (start 250.45 147) (end 250.45 142.14) (width 1) (layer F.Cu) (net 11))
 (segment (start 244.080599 140.105001) (end 243.875001 140.105001) (width 1) (layer F.Cu) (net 10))
 (segment (start 247.75 143.774402) (end 244.080599 140.105001) (width 1) (layer F.Cu) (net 10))
 (segment (start 247.75 147) (end 247.75 143.774402) (width 1) (layer F.Cu) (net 10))
 (segment (start 255.85 147) (end 255.85 151.15) (width 1) (layer F.Cu) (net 12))
 (segment (start 255.85 151.15) (end 254.2 152.8) (width 1) (layer F.Cu) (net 12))
 (segment (start 254.2 152.8) (end 225.4 152.8) (width 1) (layer F.Cu) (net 12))
 (segment (start 222.865001 150.265001) (end 221.015001 150.265001) (width 1) (layer F.Cu) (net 12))
 (segment (start 225.4 152.8) (end 222.865001 150.265001) (width 1) (layer F.Cu) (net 12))
 (segment (start 243.875001 142.645001) (end 239.154999 142.645001) (width 1) (layer B.Cu) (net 19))
 (segment (start 239.154999 142.645001) (end 227.8 154) (width 1) (layer B.Cu) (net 19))
 (segment (start 227.8 154) (end 218.2 154) (width 1) (layer B.Cu) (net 19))
 (segment (start 218.2 154) (end 214.8 150.6) (width 1) (layer B.Cu) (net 19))
 (segment (start 214.8 96.2) (end 219.6 91.4) (width 1) (layer B.Cu) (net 19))
 (segment (start 214.8 150.6) (end 214.8 96.2) (width 1) (layer B.Cu) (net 19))
 (segment (start 241.49 91.4) (end 252.965001 102.875001) (width 1) (layer F.Cu) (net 3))
 (segment (start 227.2 91.4) (end 241.49 91.4) (width 1) (layer F.Cu) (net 3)))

